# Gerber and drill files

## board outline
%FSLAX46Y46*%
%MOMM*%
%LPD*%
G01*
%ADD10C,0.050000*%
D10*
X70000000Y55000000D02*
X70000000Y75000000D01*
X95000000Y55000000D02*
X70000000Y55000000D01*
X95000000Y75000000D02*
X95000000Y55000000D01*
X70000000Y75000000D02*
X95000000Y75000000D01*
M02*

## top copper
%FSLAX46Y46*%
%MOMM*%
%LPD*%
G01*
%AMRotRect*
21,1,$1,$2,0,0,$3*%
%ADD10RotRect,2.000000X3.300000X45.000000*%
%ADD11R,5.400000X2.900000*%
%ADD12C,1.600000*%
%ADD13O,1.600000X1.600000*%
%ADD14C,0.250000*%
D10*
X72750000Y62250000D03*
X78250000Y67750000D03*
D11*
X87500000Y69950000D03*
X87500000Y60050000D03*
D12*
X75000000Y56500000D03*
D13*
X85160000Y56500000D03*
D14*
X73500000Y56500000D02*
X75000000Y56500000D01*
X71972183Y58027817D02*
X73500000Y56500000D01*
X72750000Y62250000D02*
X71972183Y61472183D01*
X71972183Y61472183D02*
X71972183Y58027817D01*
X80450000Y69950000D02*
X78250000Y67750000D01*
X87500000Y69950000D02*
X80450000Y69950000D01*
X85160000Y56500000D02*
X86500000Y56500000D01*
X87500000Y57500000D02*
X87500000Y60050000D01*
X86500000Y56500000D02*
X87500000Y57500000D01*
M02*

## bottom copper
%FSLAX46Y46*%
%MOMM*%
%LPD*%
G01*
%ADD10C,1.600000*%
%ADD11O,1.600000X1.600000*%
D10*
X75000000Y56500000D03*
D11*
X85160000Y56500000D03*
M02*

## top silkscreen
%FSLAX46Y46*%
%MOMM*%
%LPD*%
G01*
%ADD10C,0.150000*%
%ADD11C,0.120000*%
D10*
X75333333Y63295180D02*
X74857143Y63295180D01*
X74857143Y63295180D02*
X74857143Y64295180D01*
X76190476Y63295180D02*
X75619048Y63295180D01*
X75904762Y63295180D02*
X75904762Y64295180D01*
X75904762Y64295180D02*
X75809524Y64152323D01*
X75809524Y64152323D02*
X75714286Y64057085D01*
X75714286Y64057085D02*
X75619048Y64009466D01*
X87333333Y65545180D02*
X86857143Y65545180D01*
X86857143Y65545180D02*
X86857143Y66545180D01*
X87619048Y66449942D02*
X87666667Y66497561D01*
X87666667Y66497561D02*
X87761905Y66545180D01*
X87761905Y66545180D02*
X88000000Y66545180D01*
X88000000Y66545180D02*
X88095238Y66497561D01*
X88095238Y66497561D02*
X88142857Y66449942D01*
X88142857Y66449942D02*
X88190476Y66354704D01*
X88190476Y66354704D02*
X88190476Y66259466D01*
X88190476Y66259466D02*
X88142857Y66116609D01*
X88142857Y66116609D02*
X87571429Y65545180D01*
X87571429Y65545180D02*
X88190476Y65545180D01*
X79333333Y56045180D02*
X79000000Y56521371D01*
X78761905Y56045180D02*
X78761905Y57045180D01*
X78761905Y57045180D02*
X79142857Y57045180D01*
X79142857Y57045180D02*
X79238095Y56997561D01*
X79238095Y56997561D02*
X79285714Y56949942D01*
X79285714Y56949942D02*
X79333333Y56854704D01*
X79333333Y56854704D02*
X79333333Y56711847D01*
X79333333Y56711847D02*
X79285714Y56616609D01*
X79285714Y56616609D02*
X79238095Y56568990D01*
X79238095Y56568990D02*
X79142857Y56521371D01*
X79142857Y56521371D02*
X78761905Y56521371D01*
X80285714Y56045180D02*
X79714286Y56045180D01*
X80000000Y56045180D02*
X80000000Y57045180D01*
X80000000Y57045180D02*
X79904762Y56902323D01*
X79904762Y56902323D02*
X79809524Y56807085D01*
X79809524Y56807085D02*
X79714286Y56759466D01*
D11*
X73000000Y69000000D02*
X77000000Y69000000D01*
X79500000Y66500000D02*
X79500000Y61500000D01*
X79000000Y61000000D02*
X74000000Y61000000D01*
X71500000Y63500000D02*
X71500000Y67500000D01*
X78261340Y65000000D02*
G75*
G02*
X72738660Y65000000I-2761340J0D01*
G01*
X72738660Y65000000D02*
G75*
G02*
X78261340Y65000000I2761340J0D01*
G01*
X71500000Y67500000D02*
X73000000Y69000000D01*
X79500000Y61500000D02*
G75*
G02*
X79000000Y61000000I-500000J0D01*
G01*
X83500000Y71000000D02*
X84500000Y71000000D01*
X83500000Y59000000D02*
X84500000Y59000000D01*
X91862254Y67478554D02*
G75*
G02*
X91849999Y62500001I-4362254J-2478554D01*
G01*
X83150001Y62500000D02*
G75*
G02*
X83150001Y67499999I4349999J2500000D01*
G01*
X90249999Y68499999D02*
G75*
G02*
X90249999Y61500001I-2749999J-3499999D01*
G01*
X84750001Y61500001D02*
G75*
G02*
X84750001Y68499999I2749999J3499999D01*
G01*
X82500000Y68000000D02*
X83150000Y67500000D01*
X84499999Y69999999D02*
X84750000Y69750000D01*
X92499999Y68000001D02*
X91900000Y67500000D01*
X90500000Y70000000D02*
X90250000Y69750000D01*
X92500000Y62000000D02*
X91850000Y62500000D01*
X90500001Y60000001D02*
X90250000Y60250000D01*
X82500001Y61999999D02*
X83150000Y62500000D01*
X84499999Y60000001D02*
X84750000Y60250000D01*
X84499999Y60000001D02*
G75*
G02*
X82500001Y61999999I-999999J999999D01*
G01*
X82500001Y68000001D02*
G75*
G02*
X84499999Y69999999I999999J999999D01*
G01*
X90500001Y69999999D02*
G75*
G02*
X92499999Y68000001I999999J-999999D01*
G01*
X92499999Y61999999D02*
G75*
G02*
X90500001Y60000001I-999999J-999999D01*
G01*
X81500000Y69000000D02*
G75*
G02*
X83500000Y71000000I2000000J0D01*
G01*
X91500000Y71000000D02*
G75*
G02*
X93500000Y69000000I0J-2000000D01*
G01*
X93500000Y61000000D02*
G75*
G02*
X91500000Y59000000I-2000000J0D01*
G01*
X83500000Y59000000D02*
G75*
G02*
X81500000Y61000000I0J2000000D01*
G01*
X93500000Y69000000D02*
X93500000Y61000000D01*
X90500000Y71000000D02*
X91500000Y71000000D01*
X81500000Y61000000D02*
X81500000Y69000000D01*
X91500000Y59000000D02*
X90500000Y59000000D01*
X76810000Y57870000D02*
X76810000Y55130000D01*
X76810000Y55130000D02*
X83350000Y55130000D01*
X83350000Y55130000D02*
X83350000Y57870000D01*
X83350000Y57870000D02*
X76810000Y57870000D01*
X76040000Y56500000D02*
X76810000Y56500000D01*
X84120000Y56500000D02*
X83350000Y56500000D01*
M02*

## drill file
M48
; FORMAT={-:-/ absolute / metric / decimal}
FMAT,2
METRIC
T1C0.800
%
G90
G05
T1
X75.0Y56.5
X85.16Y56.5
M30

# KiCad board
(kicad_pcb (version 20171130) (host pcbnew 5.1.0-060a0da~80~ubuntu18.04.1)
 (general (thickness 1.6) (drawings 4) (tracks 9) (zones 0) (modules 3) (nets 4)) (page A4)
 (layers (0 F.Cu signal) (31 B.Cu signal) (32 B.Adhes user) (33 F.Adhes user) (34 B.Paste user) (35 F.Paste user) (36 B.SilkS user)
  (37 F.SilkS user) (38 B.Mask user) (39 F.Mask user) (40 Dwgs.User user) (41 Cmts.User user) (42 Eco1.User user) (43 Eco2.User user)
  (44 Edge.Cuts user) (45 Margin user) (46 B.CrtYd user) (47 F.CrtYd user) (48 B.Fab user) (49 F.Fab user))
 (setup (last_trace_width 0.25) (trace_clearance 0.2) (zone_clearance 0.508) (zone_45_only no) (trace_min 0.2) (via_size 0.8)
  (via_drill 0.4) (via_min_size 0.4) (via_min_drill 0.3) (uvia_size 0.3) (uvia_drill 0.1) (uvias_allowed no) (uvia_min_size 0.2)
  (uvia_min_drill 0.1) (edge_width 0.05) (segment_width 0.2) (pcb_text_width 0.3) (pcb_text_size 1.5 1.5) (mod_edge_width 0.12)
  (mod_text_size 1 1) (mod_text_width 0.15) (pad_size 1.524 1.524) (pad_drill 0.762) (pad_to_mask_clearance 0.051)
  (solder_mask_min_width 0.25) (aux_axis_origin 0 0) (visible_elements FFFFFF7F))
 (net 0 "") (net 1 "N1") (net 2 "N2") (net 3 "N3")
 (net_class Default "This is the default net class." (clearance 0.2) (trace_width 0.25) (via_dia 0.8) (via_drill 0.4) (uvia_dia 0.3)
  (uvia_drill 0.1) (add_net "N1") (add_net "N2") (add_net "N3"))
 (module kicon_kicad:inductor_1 (layer F.Cu) (at 75.5 -65)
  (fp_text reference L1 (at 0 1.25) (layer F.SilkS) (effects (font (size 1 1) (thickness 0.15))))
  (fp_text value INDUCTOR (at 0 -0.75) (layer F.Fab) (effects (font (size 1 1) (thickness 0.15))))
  (fp_line (start -2.5 -4) (end 1.5 -4) (layer F.SilkS) (width 0.12))
  (fp_line (start 4 -1.5) (end 4 3.5) (layer F.SilkS) (width 0.12))
  (fp_line (start 3.5 4) (end -1.5 4) (layer F.SilkS) (width 0.12))
  (fp_line (start -4 1.5) (end -4 -2.5) (layer F.SilkS) (width 0.12))
  (fp_circle (center 0 0) (end -2.75 0.25) (layer F.SilkS) (width 0.12))
  (fp_line (start -4 -2.5) (end -2.5 -4) (layer F.SilkS) (width 0.12))
  (fp_arc (start 3.5 3.5) (end 3.5 4) (angle -90) (layer F.SilkS) (width 0.12))
  (pad 1 smd rect (at -2.75 2.75 45) (size 2 3.3) (layers F.Cu F.Paste F.Mask) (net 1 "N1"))
  (pad 2 smd rect (at 2.75 -2.75 45) (size 2 3.3) (layers F.Cu F.Paste F.Mask) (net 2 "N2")))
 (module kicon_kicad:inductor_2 (layer F.Cu) (at 87.5 -65 180)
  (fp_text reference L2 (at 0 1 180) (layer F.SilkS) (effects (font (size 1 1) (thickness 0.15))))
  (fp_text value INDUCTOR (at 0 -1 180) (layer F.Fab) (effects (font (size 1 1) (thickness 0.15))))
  (fp_line (start 4 6) (end 3 6) (layer F.SilkS) (width 0.12))
  (fp_line (start 4 -6) (end 3 -6) (layer F.SilkS) (width 0.12))
  (fp_arc (start 0 0) (end -4.349999 -2.499999) (angle -59.49097769) (layer F.SilkS) (width 0.12))
  (fp_arc (start 0 0) (end 4.349999 2.499999) (angle -59.77305388) (layer F.SilkS) (width 0.12))
  (fp_arc (start 0 0) (end -2.749999 -3.499999) (angle -103.6855468) (layer F.SilkS) (width 0.12))
  (fp_arc (start 0 0) (end 2.749999 3.499999) (angle -103.6855468) (layer F.SilkS) (width 0.12))
  (fp_line (start 5 3) (end 4.35 2.5) (layer F.SilkS) (width 0.12))
  (fp_line (start 3.000001 4.999999) (end 2.75 4.75) (layer F.SilkS) (width 0.12))
  (fp_line (start -4.999999 3.000001) (end -4.4 2.5) (layer F.SilkS) (width 0.12))
  (fp_line (start -3 5) (end -2.75 4.75) (layer F.SilkS) (width 0.12))
  (fp_line (start -5 -3) (end -4.35 -2.5) (layer F.SilkS) (width 0.12))
  (fp_line (start -3.000001 -4.999999) (end -2.75 -4.75) (layer F.SilkS) (width 0.12))
  (fp_line (start 4.999999 -3.000001) (end 4.35 -2.5) (layer F.SilkS) (width 0.12))
  (fp_line (start 3.000001 -4.999999) (end 2.75 -4.75) (layer F.SilkS) (width 0.12))
  (fp_arc (start 4 -4) (end 4.999999 -3.000001) (angle -180) (layer F.SilkS) (width 0.12))
  (fp_arc (start 4 4) (end 3.000001 4.999999) (angle -180) (layer F.SilkS) (width 0.12))
  (fp_arc (start -4 4) (end -4.999999 3.000001) (angle -180) (layer F.SilkS) (width 0.12))
  (fp_arc (start -4 -4) (end -3.000001 -4.999999) (angle -180) (layer F.SilkS) (width 0.12))
  (fp_arc (start 4 4) (end 4 6) (angle -90) (layer F.SilkS) (width 0.12))
  (fp_arc (start -4 4) (end -6 4) (angle -90) (layer F.SilkS) (width 0.12))
  (fp_arc (start -4 -4) (end -4 -6) (angle -90) (layer F.SilkS) (width 0.12))
  (fp_arc (start 4 -4) (end 6 -4) (angle -90) (layer F.SilkS) (width 0.12))
  (fp_line (start -6 4) (end -6 -4) (layer F.SilkS) (width 0.12))
  (fp_line (start -3 6) (end -4 6) (layer F.SilkS) (width 0.12))
  (fp_line (start 6 -4) (end 6 4) (layer F.SilkS) (width 0.12))
  (fp_line (start -4 -6) (end -3 -6) (layer F.SilkS) (width 0.12))
  (pad 2 smd rect (at 0 4.95 180) (size 5.4 2.9) (layers F.Cu F.Paste F.Mask) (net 2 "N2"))
  (pad 1 smd rect (at 0 -4.95 180) (size 5.4 2.9) (layers F.Cu F.Paste F.Mask) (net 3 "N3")))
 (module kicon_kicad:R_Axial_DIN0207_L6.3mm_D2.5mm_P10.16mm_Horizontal (layer F.Cu) (at 75 -56.5)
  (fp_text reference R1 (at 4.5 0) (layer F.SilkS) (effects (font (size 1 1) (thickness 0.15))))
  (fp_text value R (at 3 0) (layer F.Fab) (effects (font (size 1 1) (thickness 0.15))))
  (fp_line (start 1.81 -1.37) (end 1.81 1.37) (layer F.SilkS) (width 0.12))
  (fp_line (start 1.81 1.37) (end 8.35 1.37) (layer F.SilkS) (width 0.12))
  (fp_line (start 8.35 1.37) (end 8.35 -1.37) (layer F.SilkS) (width 0.12))
  (fp_line (start 8.35 -1.37) (end 1.81 -1.37) (layer F.SilkS) (width 0.12))
  (fp_line (start 1.04 0) (end 1.81 0) (layer F.SilkS) (width 0.12))
  (fp_line (start 9.12 0) (end 8.35 0) (layer F.SilkS) (width 0.12))
  (pad 1 thru_hole circle (at 0 0) (size 1.6 1.6) (drill 0.8) (layers *.Cu *.Mask) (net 1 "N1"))
  (pad 2 thru_hole oval (at 10.16 0) (size 1.6 1.6) (drill 0.8) (layers *.Cu *.Mask) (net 3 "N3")))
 (gr_line (start 70 -55) (end 70 -75) (layer Edge.Cuts) (width 0.05))
 (gr_line (start 95 -55) (end 70 -55) (layer Edge.Cuts) (width 0.05))
 (gr_line (start 95 -75) (end 95 -55) (layer Edge.Cuts) (width 0.05))
 (gr_line (start 70 -75) (end 95 -75) (layer Edge.Cuts) (width 0.05))
 (segment (start 73.5 -56.5) (end 75 -56.5) (width 0.25) (layer F.Cu) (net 1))
 (segment (start 71.972183 -58.027817) (end 73.5 -56.5) (width 0.25) (layer F.Cu) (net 1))
 (segment (start 72.75 -62.25) (end 71.972183 -61.472183) (width 0.25) (layer F.Cu) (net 1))
 (segment (start 71.972183 -61.472183) (end 71.972183 -58.027817) (width 0.25) (layer F.Cu) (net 1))
 (segment (start 80.45 -69.95) (end 78.25 -67.75) (width 0.25) (layer F.Cu) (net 2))
 (segment (start 87.5 -69.95) (end 80.45 -69.95) (width 0.25) (layer F.Cu) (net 2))
 (segment (start 85.16 -56.5) (end 86.5 -56.5) (width 0.25) (layer F.Cu) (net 3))
 (segment (start 87.5 -57.5) (end 87.5 -60.05) (width 0.25) (layer F.Cu) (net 3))
 (segment (start 86.5 -56.5) (end 87.5 -57.5) (width 0.25) (layer F.Cu) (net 3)))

